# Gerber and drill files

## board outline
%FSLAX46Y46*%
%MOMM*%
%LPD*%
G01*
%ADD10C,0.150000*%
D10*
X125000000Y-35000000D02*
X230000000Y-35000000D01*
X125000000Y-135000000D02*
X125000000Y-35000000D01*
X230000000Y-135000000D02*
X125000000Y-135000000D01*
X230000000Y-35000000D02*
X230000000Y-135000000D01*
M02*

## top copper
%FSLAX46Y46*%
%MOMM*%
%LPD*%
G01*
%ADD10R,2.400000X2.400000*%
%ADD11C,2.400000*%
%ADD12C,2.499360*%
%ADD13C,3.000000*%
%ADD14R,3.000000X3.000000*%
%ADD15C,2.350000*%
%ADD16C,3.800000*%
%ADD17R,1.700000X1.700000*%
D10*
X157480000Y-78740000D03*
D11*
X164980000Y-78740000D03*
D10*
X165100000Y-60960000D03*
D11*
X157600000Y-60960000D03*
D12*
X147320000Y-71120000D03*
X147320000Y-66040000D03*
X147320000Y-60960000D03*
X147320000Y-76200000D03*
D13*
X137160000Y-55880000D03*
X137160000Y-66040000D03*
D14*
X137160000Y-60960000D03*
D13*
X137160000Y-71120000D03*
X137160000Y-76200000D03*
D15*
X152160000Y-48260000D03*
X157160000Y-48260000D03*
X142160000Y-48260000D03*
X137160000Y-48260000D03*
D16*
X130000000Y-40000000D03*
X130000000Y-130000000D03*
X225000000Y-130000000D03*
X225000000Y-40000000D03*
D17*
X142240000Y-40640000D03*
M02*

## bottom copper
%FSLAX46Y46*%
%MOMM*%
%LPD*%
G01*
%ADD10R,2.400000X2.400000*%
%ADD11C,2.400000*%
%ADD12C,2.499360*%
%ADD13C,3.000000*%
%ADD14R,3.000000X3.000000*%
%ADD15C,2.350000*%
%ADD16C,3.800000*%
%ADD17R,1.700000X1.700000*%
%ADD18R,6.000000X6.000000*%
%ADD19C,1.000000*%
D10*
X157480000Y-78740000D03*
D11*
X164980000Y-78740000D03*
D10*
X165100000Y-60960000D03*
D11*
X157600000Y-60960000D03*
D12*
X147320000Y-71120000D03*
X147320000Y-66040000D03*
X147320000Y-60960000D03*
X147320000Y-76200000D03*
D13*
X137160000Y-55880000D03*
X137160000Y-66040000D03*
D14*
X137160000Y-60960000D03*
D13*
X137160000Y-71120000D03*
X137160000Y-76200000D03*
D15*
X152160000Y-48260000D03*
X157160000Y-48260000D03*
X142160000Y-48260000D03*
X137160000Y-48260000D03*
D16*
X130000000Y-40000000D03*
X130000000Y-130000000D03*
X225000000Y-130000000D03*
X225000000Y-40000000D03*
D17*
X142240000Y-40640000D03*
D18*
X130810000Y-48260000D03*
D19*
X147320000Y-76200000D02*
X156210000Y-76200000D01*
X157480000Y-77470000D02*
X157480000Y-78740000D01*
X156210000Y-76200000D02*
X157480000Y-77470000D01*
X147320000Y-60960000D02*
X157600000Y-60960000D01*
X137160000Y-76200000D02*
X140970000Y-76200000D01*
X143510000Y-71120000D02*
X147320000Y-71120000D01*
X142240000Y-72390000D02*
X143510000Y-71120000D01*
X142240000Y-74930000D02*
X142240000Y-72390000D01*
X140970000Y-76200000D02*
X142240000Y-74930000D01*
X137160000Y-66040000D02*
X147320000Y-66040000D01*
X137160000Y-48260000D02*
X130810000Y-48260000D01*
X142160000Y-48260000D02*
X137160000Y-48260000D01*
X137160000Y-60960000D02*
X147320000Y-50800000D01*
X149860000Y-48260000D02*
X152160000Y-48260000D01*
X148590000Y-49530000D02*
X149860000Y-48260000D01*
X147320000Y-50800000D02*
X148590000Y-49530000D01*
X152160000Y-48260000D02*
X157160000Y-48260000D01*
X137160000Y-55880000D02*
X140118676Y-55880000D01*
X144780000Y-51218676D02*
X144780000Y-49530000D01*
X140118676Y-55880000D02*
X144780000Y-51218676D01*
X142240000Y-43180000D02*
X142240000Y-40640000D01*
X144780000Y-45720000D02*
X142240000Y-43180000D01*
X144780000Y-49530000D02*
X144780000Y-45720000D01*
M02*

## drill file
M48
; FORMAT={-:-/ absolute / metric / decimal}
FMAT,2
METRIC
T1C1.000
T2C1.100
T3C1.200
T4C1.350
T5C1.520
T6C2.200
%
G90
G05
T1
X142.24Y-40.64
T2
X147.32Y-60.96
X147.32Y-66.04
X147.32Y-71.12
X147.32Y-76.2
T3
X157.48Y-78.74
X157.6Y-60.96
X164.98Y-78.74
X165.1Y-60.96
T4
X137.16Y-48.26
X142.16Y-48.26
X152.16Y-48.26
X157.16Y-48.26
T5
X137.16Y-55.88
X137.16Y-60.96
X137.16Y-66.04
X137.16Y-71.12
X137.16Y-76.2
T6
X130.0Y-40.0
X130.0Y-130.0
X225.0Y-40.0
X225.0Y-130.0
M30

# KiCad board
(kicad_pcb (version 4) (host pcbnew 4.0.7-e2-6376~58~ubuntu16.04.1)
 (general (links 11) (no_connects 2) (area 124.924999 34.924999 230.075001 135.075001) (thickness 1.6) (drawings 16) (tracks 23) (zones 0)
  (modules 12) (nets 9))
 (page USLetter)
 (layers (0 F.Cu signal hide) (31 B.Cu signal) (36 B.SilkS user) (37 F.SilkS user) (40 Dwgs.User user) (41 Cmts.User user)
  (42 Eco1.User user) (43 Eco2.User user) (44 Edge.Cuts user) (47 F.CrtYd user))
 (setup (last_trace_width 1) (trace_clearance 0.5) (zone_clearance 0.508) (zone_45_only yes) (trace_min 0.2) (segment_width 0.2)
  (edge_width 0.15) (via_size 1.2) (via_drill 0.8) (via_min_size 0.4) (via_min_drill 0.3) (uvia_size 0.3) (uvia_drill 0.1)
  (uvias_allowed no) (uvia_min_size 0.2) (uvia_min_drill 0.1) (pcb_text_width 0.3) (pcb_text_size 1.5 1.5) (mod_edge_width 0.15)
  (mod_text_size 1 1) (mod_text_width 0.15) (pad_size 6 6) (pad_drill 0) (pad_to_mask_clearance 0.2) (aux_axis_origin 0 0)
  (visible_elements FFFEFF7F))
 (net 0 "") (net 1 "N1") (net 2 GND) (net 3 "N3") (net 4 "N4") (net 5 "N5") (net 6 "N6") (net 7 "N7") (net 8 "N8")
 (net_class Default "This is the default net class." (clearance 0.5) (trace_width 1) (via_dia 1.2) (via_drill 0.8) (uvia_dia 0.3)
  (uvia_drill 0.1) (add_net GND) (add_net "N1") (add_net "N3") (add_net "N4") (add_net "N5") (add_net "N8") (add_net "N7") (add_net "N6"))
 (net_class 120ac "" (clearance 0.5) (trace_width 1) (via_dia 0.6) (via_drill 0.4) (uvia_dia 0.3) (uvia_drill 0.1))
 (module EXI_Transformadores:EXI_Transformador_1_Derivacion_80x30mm (layer F.Cu) (at 85 85 90)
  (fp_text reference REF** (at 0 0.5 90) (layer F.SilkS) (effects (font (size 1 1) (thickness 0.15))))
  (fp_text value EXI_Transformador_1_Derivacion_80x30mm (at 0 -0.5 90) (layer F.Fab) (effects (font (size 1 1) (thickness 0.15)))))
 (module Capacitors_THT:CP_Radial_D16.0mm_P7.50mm (layer F.Cu) (at 157.48 78.74)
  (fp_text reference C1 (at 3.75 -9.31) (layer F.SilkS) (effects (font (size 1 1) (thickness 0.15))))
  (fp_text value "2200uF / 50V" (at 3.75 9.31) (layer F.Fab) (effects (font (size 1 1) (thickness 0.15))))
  (pad 1 thru_hole rect (at 0 0) (size 2.4 2.4) (drill 1.2) (layers *.Cu *.Mask) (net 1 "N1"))
  (pad 2 thru_hole circle (at 7.5 0) (size 2.4 2.4) (drill 1.2) (layers *.Cu *.Mask) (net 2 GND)))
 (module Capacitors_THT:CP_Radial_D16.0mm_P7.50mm (layer F.Cu) (at 165.1 60.96 180)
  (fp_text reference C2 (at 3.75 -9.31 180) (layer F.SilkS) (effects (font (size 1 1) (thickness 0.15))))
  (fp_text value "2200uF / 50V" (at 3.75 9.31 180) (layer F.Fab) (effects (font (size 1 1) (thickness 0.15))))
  (pad 1 thru_hole rect (at 0 0 180) (size 2.4 2.4) (drill 1.2) (layers *.Cu *.Mask) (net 2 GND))
  (pad 2 thru_hole circle (at 7.5 0 180) (size 2.4 2.4) (drill 1.2) (layers *.Cu *.Mask) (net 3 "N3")))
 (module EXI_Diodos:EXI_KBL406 (layer F.Cu) (at 147.32 68.58 90)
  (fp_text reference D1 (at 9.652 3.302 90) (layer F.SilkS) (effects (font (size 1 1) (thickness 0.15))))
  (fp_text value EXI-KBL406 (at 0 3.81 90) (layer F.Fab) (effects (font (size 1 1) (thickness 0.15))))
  (pad 2 thru_hole circle (at -2.54 0 90) (size 2.49936 2.49936) (drill 1.09982) (layers *.Cu *.Mask F.SilkS) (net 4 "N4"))
  (pad 3 thru_hole circle (at 2.54 0 90) (size 2.49936 2.49936) (drill 1.09982) (layers *.Cu *.Mask F.SilkS) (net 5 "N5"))
  (pad 4 thru_hole circle (at 7.62 0 90) (size 2.49936 2.49936) (drill 1.09982) (layers *.Cu *.Mask F.SilkS) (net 3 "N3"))
  (pad 1 thru_hole circle (at -7.62 0 90) (size 2.49936 2.49936) (drill 1.09982) (layers *.Cu *.Mask F.SilkS) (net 1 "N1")))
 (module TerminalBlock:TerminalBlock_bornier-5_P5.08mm (layer F.Cu) (at 137.16 76.2 90)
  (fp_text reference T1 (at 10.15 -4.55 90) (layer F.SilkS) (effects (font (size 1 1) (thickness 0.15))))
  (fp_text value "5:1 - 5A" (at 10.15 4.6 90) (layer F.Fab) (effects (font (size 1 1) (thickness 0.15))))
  (pad 2 thru_hole circle (at 20.32 0 90) (size 3 3) (drill 1.52) (layers *.Cu *.Mask) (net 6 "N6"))
  (pad 3 thru_hole circle (at 10.16 0 90) (size 3 3) (drill 1.52) (layers *.Cu *.Mask) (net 5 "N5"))
  (pad 1 thru_hole rect (at 15.24 0 90) (size 3 3) (drill 1.52) (layers *.Cu *.Mask) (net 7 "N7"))
  (pad 4 thru_hole circle (at 5.08 0 90) (size 3 3) (drill 1.52) (layers *.Cu *.Mask) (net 2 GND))
  (pad 5 thru_hole circle (at 0 0 90) (size 3 3) (drill 1.52) (layers *.Cu *.Mask) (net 4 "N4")))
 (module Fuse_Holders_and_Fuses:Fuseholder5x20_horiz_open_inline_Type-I (layer F.Cu) (at 137.16 48.26)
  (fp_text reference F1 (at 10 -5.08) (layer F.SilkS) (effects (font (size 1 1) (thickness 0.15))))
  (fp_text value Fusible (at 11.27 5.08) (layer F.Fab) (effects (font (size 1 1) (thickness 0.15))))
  (pad 2 thru_hole circle (at 15 0) (size 2.35 2.35) (drill 1.35) (layers *.Cu *.Mask) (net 7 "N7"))
  (pad 2 thru_hole circle (at 20 0) (size 2.35 2.35) (drill 1.35) (layers *.Cu *.Mask) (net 7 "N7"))
  (pad 1 thru_hole circle (at 5 0) (size 2.35 2.35) (drill 1.35) (layers *.Cu *.Mask) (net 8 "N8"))
  (pad 1 thru_hole circle (at 0 0) (size 2.35 2.35) (drill 1.35) (layers *.Cu *.Mask) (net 8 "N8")))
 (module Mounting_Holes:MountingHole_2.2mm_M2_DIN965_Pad (layer F.Cu) (at 130 40)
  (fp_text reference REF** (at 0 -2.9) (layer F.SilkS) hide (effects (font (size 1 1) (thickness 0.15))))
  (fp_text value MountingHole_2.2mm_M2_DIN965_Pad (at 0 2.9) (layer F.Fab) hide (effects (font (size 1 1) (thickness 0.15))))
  (pad 1 thru_hole circle (at 0 0) (size 3.8 3.8) (drill 2.2) (layers *.Cu *.Mask)))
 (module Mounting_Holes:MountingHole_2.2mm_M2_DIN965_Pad (layer F.Cu) (at 130 130)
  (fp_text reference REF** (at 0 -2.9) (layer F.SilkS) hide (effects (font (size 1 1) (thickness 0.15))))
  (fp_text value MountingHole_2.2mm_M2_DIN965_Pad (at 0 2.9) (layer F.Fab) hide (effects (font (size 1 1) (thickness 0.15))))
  (pad 1 thru_hole circle (at 0 0) (size 3.8 3.8) (drill 2.2) (layers *.Cu *.Mask)))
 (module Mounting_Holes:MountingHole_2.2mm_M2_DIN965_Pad (layer F.Cu) (at 225 130)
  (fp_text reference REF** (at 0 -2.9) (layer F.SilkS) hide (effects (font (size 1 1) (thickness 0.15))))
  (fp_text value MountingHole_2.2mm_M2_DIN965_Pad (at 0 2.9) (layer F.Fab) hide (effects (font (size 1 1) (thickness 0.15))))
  (pad 1 thru_hole circle (at 0 0) (size 3.8 3.8) (drill 2.2) (layers *.Cu *.Mask)))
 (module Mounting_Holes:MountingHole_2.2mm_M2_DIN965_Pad (layer F.Cu) (at 225 40)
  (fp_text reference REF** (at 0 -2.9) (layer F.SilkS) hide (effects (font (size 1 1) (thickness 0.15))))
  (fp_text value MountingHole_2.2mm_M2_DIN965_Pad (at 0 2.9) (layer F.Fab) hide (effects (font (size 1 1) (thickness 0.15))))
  (pad 1 thru_hole circle (at 0 0) (size 3.8 3.8) (drill 2.2) (layers *.Cu *.Mask)))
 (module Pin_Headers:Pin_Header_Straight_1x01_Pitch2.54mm (layer F.Cu) (at 142.24 40.64)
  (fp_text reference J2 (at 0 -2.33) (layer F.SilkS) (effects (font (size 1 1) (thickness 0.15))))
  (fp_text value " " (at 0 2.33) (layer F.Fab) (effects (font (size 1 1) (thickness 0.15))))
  (pad 1 thru_hole rect (at 0 0) (size 1.7 1.7) (drill 1) (layers *.Cu *.Mask) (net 6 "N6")))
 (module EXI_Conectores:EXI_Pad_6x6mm (layer B.Cu) (at 130.81 48.26 90)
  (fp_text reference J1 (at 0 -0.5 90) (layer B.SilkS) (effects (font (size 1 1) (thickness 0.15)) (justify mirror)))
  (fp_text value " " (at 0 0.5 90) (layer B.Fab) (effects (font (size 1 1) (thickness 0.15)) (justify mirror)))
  (pad 1 smd rect (at 0 0 90) (size 6 6) (layers B.Cu) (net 8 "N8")))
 (gr_line (start 125 35) (end 230 35) (angle 90) (layer Edge.Cuts) (width 0.15))
 (gr_line (start 125 135) (end 125 35) (angle 90) (layer Edge.Cuts) (width 0.15))
 (gr_line (start 230 135) (end 125 135) (angle 90) (layer Edge.Cuts) (width 0.15))
 (gr_line (start 230 35) (end 230 135) (angle 90) (layer Edge.Cuts) (width 0.15))
 (segment (start 147.32 76.2) (end 156.21 76.2) (width 1) (layer B.Cu) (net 1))
 (segment (start 157.48 77.47) (end 157.48 78.74) (width 1) (layer B.Cu) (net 1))
 (segment (start 156.21 76.2) (end 157.48 77.47) (width 1) (layer B.Cu) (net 1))
 (segment (start 147.32 60.96) (end 157.6 60.96) (width 1) (layer B.Cu) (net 3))
 (segment (start 137.16 76.2) (end 140.97 76.2) (width 1) (layer B.Cu) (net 4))
 (segment (start 143.51 71.12) (end 147.32 71.12) (width 1) (layer B.Cu) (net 4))
 (segment (start 142.24 72.39) (end 143.51 71.12) (width 1) (layer B.Cu) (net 4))
 (segment (start 142.24 74.93) (end 142.24 72.39) (width 1) (layer B.Cu) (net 4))
 (segment (start 140.97 76.2) (end 142.24 74.93) (width 1) (layer B.Cu) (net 4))
 (segment (start 137.16 66.04) (end 147.32 66.04) (width 1) (layer B.Cu) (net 5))
 (segment (start 137.16 48.26) (end 130.81 48.26) (width 1) (layer B.Cu) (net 8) (status C00000))
 (segment (start 142.16 48.26) (end 137.16 48.26) (width 1) (layer B.Cu) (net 8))
 (segment (start 137.16 60.96) (end 147.32 50.8) (width 1) (layer B.Cu) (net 7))
 (segment (start 149.86 48.26) (end 152.16 48.26) (width 1) (layer B.Cu) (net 7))
 (segment (start 148.59 49.53) (end 149.86 48.26) (width 1) (layer B.Cu) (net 7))
 (segment (start 147.32 50.8) (end 148.59 49.53) (width 1) (layer B.Cu) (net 7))
 (segment (start 152.16 48.26) (end 157.16 48.26) (width 1) (layer B.Cu) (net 7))
 (segment (start 137.16 55.88) (end 140.118676 55.88) (width 1) (layer B.Cu) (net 6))
 (segment (start 144.78 51.218676) (end 144.78 49.53) (width 1) (layer B.Cu) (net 6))
 (segment (start 140.118676 55.88) (end 144.78 51.218676) (width 1) (layer B.Cu) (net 6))
 (segment (start 142.24 43.18) (end 142.24 40.64) (width 1) (layer B.Cu) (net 6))
 (segment (start 144.78 45.72) (end 142.24 43.18) (width 1) (layer B.Cu) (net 6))
 (segment (start 144.78 49.53) (end 144.78 45.72) (width 1) (layer B.Cu) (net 6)))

